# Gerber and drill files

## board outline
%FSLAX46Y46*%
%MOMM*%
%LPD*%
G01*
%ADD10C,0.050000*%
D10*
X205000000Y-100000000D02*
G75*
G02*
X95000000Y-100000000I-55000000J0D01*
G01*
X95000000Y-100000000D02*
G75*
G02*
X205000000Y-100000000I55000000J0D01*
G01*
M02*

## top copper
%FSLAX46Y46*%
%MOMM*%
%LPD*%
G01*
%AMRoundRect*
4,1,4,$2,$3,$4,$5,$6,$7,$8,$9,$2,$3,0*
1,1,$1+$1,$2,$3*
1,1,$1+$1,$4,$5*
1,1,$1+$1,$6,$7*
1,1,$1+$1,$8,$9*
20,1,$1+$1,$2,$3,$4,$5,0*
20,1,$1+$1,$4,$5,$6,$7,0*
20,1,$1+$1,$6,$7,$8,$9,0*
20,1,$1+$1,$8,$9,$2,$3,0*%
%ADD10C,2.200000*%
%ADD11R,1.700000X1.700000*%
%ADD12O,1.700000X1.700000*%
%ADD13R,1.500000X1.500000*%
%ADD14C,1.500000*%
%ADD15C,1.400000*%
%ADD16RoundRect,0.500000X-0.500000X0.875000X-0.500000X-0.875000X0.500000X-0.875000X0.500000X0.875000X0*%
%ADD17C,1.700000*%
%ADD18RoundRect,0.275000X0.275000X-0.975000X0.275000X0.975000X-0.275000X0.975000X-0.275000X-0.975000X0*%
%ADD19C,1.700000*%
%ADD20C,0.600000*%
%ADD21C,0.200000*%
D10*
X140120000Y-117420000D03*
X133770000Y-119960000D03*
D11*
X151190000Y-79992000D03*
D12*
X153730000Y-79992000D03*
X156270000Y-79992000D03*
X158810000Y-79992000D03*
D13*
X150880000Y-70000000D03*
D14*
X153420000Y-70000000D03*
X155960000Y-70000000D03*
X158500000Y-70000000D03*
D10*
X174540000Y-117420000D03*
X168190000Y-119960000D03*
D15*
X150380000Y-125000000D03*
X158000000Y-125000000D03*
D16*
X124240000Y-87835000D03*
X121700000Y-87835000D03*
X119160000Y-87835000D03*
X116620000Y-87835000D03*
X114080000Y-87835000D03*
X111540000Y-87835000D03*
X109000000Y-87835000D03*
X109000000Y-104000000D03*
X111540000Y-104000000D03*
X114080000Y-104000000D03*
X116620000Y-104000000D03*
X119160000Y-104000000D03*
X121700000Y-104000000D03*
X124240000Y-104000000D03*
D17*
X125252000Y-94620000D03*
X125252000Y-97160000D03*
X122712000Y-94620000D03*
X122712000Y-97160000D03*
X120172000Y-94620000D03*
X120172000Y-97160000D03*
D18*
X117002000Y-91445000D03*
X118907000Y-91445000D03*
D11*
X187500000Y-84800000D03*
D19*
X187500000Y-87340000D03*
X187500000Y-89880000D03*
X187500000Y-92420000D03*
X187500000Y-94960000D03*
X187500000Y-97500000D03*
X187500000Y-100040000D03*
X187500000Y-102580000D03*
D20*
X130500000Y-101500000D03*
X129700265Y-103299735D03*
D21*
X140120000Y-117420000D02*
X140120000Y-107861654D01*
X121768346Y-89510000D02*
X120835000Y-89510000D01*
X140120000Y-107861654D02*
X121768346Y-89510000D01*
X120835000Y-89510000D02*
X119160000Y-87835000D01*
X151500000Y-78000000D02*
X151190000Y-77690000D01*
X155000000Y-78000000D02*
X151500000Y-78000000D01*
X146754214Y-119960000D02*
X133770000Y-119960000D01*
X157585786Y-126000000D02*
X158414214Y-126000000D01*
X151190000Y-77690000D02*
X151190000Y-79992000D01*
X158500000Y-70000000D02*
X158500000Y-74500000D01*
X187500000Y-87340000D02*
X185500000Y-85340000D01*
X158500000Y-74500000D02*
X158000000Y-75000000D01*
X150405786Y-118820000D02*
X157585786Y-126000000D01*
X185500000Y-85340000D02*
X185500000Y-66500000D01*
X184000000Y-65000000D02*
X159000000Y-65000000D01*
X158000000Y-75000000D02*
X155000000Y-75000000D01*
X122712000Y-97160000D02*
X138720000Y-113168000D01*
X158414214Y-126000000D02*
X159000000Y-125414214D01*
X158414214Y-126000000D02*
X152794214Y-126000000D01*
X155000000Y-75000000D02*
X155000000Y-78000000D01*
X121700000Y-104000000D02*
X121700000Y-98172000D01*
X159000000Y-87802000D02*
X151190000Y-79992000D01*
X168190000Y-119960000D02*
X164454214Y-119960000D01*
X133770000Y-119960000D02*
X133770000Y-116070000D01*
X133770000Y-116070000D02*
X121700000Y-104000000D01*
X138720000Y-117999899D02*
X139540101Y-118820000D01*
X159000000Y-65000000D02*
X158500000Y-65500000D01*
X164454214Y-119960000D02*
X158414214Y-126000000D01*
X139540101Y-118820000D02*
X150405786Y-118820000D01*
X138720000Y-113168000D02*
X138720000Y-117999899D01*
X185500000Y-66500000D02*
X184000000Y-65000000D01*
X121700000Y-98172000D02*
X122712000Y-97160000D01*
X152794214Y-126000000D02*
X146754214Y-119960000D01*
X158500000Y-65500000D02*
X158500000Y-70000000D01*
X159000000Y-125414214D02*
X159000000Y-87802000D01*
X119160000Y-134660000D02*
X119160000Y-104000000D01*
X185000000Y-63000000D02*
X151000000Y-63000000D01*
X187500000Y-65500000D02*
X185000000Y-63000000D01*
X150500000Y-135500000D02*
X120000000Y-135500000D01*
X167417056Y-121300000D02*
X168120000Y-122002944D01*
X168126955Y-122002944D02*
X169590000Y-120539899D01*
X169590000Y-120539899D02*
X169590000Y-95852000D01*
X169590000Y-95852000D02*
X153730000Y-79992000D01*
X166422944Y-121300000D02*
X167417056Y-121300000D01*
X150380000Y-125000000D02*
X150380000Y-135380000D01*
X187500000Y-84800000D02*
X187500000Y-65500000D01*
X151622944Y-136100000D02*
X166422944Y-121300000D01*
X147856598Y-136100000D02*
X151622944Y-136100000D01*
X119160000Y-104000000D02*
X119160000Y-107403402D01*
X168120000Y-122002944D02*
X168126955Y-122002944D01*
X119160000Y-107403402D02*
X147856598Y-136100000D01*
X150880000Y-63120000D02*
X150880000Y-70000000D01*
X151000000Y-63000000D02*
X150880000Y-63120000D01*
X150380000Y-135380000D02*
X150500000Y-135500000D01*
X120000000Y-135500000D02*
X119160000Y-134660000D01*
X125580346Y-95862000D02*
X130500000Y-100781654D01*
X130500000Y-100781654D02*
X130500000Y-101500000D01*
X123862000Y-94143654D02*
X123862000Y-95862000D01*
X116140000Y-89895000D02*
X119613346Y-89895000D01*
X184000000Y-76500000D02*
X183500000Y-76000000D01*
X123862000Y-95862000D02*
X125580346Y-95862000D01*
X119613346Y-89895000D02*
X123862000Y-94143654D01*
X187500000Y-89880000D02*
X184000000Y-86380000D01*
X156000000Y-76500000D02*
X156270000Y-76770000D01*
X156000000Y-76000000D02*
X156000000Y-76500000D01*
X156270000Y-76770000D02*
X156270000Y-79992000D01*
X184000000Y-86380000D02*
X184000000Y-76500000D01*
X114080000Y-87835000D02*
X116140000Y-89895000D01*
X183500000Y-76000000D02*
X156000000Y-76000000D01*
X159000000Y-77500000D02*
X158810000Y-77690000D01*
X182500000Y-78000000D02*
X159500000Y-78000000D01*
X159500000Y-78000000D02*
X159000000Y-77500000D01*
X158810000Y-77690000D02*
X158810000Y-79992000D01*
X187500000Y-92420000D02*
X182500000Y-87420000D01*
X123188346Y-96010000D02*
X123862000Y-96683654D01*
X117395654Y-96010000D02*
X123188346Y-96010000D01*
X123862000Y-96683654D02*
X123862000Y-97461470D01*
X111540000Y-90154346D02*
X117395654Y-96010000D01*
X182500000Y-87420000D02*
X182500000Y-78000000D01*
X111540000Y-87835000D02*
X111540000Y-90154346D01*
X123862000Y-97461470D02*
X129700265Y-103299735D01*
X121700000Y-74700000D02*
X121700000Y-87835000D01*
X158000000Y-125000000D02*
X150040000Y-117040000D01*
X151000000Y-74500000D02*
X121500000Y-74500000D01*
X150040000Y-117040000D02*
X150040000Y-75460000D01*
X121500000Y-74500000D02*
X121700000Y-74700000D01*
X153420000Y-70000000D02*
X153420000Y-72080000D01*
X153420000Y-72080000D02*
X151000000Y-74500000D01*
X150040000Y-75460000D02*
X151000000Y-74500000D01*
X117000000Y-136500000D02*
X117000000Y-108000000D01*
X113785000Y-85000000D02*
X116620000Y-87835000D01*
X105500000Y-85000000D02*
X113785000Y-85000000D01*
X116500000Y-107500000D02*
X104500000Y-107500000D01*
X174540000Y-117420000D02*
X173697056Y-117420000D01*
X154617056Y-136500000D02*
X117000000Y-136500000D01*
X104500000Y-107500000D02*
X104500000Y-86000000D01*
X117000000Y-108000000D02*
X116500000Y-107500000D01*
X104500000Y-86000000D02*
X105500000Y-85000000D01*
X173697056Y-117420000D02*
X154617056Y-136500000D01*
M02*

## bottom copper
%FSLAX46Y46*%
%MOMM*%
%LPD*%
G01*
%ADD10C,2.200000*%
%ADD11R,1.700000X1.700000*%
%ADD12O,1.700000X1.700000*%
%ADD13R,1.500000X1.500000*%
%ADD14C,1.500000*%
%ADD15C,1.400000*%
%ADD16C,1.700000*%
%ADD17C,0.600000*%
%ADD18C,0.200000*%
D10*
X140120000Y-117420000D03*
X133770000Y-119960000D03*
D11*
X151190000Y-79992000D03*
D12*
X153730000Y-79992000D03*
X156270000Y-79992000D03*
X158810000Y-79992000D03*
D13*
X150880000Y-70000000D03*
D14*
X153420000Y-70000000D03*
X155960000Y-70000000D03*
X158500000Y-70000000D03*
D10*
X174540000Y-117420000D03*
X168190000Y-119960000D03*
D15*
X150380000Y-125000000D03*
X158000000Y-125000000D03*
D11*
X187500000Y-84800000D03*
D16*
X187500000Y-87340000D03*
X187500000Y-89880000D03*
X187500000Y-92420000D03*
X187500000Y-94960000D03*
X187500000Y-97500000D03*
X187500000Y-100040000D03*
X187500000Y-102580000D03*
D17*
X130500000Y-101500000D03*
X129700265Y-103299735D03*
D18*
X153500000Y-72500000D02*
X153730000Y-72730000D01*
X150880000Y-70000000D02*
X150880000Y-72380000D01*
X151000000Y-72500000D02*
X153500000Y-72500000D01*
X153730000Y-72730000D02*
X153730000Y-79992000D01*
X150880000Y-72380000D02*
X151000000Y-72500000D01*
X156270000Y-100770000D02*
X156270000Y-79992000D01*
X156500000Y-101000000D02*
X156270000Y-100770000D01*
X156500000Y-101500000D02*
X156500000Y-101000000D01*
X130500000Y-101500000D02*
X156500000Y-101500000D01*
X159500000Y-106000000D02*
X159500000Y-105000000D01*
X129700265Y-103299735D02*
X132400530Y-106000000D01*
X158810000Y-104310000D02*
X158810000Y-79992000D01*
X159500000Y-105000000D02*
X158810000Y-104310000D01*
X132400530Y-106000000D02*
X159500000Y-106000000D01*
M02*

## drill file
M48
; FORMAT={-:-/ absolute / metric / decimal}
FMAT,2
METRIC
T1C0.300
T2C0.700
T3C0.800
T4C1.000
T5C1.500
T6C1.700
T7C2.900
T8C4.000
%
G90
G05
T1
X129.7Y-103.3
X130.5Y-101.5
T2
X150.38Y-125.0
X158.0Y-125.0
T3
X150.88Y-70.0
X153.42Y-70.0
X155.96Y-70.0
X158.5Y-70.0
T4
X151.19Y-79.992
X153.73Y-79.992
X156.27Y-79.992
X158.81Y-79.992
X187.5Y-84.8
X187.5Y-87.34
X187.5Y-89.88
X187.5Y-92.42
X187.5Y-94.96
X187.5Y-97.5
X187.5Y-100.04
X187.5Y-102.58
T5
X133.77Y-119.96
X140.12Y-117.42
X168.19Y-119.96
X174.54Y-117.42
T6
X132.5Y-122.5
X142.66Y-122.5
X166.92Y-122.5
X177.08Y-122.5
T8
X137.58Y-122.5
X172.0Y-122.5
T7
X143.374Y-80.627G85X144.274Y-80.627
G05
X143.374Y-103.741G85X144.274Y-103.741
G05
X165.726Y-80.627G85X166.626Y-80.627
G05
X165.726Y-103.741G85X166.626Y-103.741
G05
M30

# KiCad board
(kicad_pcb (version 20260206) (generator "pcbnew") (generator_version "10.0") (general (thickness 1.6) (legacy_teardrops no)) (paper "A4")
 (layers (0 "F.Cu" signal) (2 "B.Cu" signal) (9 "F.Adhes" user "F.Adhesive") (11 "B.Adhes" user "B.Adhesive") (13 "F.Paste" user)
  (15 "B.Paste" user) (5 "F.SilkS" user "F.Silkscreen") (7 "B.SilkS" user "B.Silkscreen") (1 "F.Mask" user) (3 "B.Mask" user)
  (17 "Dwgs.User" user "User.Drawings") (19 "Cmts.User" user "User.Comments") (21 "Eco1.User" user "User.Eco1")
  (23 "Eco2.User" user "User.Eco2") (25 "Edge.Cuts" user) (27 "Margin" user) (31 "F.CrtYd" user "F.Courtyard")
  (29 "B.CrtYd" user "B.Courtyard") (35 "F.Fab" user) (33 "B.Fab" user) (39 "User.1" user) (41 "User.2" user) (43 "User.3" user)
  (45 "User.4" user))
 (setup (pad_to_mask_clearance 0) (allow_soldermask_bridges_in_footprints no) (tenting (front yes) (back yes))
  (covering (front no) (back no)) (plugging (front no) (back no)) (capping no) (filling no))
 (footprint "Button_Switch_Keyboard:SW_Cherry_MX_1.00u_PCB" (layer "F.Cu") (at 140.12 117.42)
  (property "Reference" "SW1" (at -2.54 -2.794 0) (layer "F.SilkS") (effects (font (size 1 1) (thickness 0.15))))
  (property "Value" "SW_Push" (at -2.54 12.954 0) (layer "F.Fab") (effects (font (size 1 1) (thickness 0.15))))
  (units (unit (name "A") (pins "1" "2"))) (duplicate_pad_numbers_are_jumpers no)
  (pad "" np_thru_hole circle (at -7.62 5.08) (size 1.7 1.7) (drill 1.7) (layers "*.Cu" "*.Mask"))
  (pad "" np_thru_hole circle (at -2.54 5.08) (size 4 4) (drill 4) (layers "*.Cu" "*.Mask"))
  (pad "" np_thru_hole circle (at 2.54 5.08) (size 1.7 1.7) (drill 1.7) (layers "*.Cu" "*.Mask"))
  (pad "1" thru_hole circle (at 0 0) (size 2.2 2.2) (drill 1.5) (layers "*.Cu" "*.Mask") (remove_unused_layers no) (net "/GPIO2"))
  (pad "2" thru_hole circle (at -6.35 2.54) (size 2.2 2.2) (drill 1.5) (layers "*.Cu" "*.Mask") (remove_unused_layers no) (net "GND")))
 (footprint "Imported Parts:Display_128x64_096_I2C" (layer "F.Cu") (at 155 79.992)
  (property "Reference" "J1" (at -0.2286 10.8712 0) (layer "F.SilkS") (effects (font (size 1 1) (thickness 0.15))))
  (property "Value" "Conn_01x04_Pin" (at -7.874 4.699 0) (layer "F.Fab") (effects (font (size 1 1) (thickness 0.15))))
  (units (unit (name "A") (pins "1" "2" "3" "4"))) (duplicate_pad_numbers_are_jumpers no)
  (pad "" np_thru_hole oval (at -11.176 0.635) (size 3.8 2.9) (drill oval 3.8 2.9) (layers "*.Cu" "*.Mask"))
  (pad "" np_thru_hole oval (at -11.176 23.749) (size 3.8 2.9) (drill oval 3.8 2.9) (layers "*.Cu" "*.Mask"))
  (pad "" np_thru_hole oval (at 11.176 0.635) (size 3.8 2.9) (drill oval 3.8 2.9) (layers "*.Cu" "*.Mask"))
  (pad "" np_thru_hole oval (at 11.176 23.749) (size 3.8 2.9) (drill oval 3.8 2.9) (layers "*.Cu" "*.Mask"))
  (pad "1" thru_hole rect (at -3.81 0 90) (size 1.7 1.7) (drill 1) (layers "*.Cu" "*.Mask") (remove_unused_layers no) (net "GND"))
  (pad "2" thru_hole oval (at -1.27 0 90) (size 1.7 1.7) (drill 1) (layers "*.Cu" "*.Mask") (remove_unused_layers no) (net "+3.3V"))
  (pad "3" thru_hole oval (at 1.27 0 90) (size 1.7 1.7) (drill 1) (layers "*.Cu" "*.Mask") (remove_unused_layers no) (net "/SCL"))
  (pad "4" thru_hole oval (at 3.81 0 90) (size 1.7 1.7) (drill 1) (layers "*.Cu" "*.Mask") (remove_unused_layers no) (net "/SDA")))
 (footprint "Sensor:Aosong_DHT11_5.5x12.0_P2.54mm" (layer "F.Cu") (at 150.88 70 90)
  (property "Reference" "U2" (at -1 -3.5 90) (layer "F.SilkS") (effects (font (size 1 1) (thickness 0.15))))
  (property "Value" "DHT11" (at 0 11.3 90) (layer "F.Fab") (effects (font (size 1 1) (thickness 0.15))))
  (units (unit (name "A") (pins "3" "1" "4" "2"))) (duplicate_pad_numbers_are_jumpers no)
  (pad "1" thru_hole rect (at 0 0 90) (size 1.5 1.5) (drill 0.8) (layers "*.Cu" "*.Mask") (remove_unused_layers no) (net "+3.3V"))
  (pad "2" thru_hole circle (at 0 2.54 90) (size 1.5 1.5) (drill 0.8) (layers "*.Cu" "*.Mask") (remove_unused_layers no) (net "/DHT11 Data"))
  (pad "3" thru_hole circle (at 0 5.08 90) (size 1.5 1.5) (drill 0.8) (layers "*.Cu" "*.Mask") (remove_unused_layers no)
   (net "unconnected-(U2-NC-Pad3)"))
  (pad "4" thru_hole circle (at 0 7.62 90) (size 1.5 1.5) (drill 0.8) (layers "*.Cu" "*.Mask") (remove_unused_layers no) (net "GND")))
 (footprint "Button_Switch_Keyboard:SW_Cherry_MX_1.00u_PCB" (layer "F.Cu") (at 174.54 117.42)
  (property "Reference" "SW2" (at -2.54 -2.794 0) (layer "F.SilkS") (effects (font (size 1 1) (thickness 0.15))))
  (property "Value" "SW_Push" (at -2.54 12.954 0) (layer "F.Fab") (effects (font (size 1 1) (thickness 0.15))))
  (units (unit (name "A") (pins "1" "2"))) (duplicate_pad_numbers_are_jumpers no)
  (pad "" np_thru_hole circle (at -7.62 5.08) (size 1.7 1.7) (drill 1.7) (layers "*.Cu" "*.Mask"))
  (pad "" np_thru_hole circle (at -2.54 5.08) (size 4 4) (drill 4) (layers "*.Cu" "*.Mask"))
  (pad "" np_thru_hole circle (at 2.54 5.08) (size 1.7 1.7) (drill 1.7) (layers "*.Cu" "*.Mask"))
  (pad "1" thru_hole circle (at 0 0) (size 2.2 2.2) (drill 1.5) (layers "*.Cu" "*.Mask") (remove_unused_layers no) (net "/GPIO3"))
  (pad "2" thru_hole circle (at -6.35 2.54) (size 2.2 2.2) (drill 1.5) (layers "*.Cu" "*.Mask") (remove_unused_layers no) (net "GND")))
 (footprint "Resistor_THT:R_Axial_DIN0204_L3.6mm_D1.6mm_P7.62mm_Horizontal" (layer "F.Cu") (at 150.38 125)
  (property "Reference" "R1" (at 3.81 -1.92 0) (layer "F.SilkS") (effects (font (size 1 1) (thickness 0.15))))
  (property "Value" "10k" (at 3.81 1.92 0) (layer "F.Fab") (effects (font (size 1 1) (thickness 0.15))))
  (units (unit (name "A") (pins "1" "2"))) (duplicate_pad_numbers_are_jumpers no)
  (pad "1" thru_hole circle (at 0 0) (size 1.4 1.4) (drill 0.7) (layers "*.Cu" "*.Mask") (remove_unused_layers no) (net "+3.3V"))
  (pad "2" thru_hole circle (at 7.62 0) (size 1.4 1.4) (drill 0.7) (layers "*.Cu" "*.Mask") (remove_unused_layers no) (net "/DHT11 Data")))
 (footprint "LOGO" (layer "F.Cu") (at 133 62)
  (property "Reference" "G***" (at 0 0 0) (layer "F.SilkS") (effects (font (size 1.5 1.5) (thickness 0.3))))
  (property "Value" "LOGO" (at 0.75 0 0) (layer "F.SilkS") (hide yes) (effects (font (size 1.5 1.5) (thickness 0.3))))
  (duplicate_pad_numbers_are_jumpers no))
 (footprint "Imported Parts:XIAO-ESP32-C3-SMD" (layer "F.Cu") (at 106.12 87 -90)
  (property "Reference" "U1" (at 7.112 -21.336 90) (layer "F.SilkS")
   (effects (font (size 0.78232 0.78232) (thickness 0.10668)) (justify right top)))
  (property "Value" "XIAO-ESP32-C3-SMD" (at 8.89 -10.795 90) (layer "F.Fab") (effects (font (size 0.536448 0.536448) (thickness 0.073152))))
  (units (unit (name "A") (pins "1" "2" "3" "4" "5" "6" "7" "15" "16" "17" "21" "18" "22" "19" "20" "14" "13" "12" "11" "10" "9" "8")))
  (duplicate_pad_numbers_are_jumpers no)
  (pad "1" smd roundrect (at 0.835 -18.12 270) (size 2.75 2) (layers "F.Cu" "F.Mask" "F.Paste") (roundrect_rratio 0.25)
   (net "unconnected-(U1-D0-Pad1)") (solder_mask_margin 0.0508) (thermal_bridge_angle 45))
  (pad "2" smd roundrect (at 0.835 -15.58 270) (size 2.75 2) (layers "F.Cu" "F.Mask" "F.Paste") (roundrect_rratio 0.25) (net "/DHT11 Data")
   (solder_mask_margin 0.0508) (thermal_bridge_angle 45))
  (pad "3" smd roundrect (at 0.835 -13.04 270) (size 2.75 2) (layers "F.Cu" "F.Mask" "F.Paste") (roundrect_rratio 0.25) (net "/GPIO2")
   (solder_mask_margin 0.0508) (thermal_bridge_angle 45))
  (pad "4" smd roundrect (at 0.835 -10.5 270) (size 2.75 2) (layers "F.Cu" "F.Mask" "F.Paste") (roundrect_rratio 0.25) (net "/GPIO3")
   (solder_mask_margin 0.0508) (thermal_bridge_angle 45))
  (pad "5" smd roundrect (at 0.835 -7.96 270) (size 2.75 2) (layers "F.Cu" "F.Mask" "F.Paste") (roundrect_rratio 0.25) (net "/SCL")
   (solder_mask_margin 0.0508) (thermal_bridge_angle 45))
  (pad "6" smd roundrect (at 0.835 -5.42 270) (size 2.75 2) (layers "F.Cu" "F.Mask" "F.Paste") (roundrect_rratio 0.25) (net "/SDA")
   (solder_mask_margin 0.0508) (thermal_bridge_angle 45))
  (pad "7" smd roundrect (at 0.835 -2.88 270) (size 2.75 2) (layers "F.Cu" "F.Mask" "F.Paste") (roundrect_rratio 0.25)
   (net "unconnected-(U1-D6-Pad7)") (solder_mask_margin 0.0508) (thermal_bridge_angle 45))
  (pad "8" smd roundrect (at 17 -2.88 270) (size 2.75 2) (layers "F.Cu" "F.Mask" "F.Paste") (roundrect_rratio 0.25)
   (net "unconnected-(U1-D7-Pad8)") (solder_mask_margin 0.0508) (thermal_bridge_angle 45))
  (pad "9" smd roundrect (at 17 -5.42 270) (size 2.75 2) (layers "F.Cu" "F.Mask" "F.Paste") (roundrect_rratio 0.25)
   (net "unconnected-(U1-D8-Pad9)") (solder_mask_margin 0.0508) (thermal_bridge_angle 45))
  (pad "10" smd roundrect (at 17 -7.96 270) (size 2.75 2) (layers "F.Cu" "F.Mask" "F.Paste") (roundrect_rratio 0.25)
   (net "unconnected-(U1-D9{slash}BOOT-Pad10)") (solder_mask_margin 0.0508) (thermal_bridge_angle 45))
  (pad "11" smd roundrect (at 17 -10.5 270) (size 2.75 2) (layers "F.Cu" "F.Mask" "F.Paste") (roundrect_rratio 0.25)
   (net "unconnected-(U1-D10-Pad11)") (solder_mask_margin 0.0508) (thermal_bridge_angle 45))
  (pad "12" smd roundrect (at 17 -13.04 270) (size 2.75 2) (layers "F.Cu" "F.Mask" "F.Paste") (roundrect_rratio 0.25) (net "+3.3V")
   (solder_mask_margin 0.0508) (thermal_bridge_angle 45))
  (pad "13" smd roundrect (at 17 -15.58 270) (size 2.75 2) (layers "F.Cu" "F.Mask" "F.Paste") (roundrect_rratio 0.25) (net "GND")
   (solder_mask_margin 0.0508) (thermal_bridge_angle 45))
  (pad "14" smd roundrect (at 17 -18.12 270) (size 2.75 2) (layers "F.Cu" "F.Mask" "F.Paste") (roundrect_rratio 0.25) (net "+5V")
   (solder_mask_margin 0.0508) (thermal_bridge_angle 45))
  (pad "15" smd circle (at 7.62 -19.132 270) (size 1.7 1.7) (layers "F.Cu" "F.Mask" "F.Paste") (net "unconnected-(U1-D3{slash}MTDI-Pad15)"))
  (pad "16" smd circle (at 10.16 -19.132 270) (size 1.7 1.7) (layers "F.Cu" "F.Mask" "F.Paste") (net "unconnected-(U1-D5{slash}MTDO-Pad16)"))
  (pad "17" smd circle (at 7.62 -16.592 270) (size 1.7 1.7) (layers "F.Cu" "F.Mask" "F.Paste") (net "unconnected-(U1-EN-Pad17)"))
  (pad "18" smd circle (at 10.16 -16.592 270) (size 1.7 1.7) (layers "F.Cu" "F.Mask" "F.Paste") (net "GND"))
  (pad "19" smd circle (at 7.62 -14.052 270) (size 1.7 1.7) (layers "F.Cu" "F.Mask" "F.Paste") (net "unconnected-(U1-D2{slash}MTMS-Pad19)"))
  (pad "20" smd circle (at 10.16 -14.052 270) (size 1.7 1.7) (layers "F.Cu" "F.Mask" "F.Paste") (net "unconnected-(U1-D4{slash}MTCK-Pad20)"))
  (pad "21" smd roundrect (at 4.445 -10.882 90) (size 2.5 1.1) (layers "F.Cu" "F.Mask" "F.Paste") (roundrect_rratio 0.25)
   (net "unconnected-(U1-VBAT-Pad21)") (thermal_bridge_angle 45))
  (pad "22" smd roundrect (at 4.445 -12.787 90) (size 2.5 1.1) (layers "F.Cu" "F.Mask" "F.Paste") (roundrect_rratio 0.25)
   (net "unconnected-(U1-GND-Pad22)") (thermal_bridge_angle 45)))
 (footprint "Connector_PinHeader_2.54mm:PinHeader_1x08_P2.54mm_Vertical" (layer "F.Cu") (at 187.5 84.8)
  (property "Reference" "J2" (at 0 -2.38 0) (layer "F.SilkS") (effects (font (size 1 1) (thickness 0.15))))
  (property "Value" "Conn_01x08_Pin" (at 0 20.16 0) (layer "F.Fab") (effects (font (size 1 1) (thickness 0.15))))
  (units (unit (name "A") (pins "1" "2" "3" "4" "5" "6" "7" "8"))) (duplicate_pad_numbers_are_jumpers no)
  (pad "1" thru_hole rect (at 0 0) (size 1.7 1.7) (drill 1) (layers "*.Cu" "*.Mask") (remove_unused_layers no) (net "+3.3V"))
  (pad "2" thru_hole circle (at 0 2.54) (size 1.7 1.7) (drill 1) (layers "*.Cu" "*.Mask") (remove_unused_layers no) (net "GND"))
  (pad "3" thru_hole circle (at 0 5.08) (size 1.7 1.7) (drill 1) (layers "*.Cu" "*.Mask") (remove_unused_layers no) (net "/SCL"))
  (pad "4" thru_hole circle (at 0 7.62) (size 1.7 1.7) (drill 1) (layers "*.Cu" "*.Mask") (remove_unused_layers no) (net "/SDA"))
  (pad "5" thru_hole circle (at 0 10.16) (size 1.7 1.7) (drill 1) (layers "*.Cu" "*.Mask") (remove_unused_layers no)
   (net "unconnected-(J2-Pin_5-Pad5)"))
  (pad "6" thru_hole circle (at 0 12.7) (size 1.7 1.7) (drill 1) (layers "*.Cu" "*.Mask") (remove_unused_layers no)
   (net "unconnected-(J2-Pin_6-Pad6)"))
  (pad "7" thru_hole circle (at 0 15.24) (size 1.7 1.7) (drill 1) (layers "*.Cu" "*.Mask") (remove_unused_layers no)
   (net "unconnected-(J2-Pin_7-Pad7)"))
  (pad "8" thru_hole circle (at 0 17.78) (size 1.7 1.7) (drill 1) (layers "*.Cu" "*.Mask") (remove_unused_layers no)
   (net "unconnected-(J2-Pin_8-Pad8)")))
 (gr_circle (center 150 100) (end 205 100) (stroke (width 0.05) (type solid)) (fill no) (layer "Edge.Cuts"))
 (segment (start 140.12 117.42) (end 140.12 107.861654) (width 0.2) (layer "F.Cu") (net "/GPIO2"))
 (segment (start 121.768346 89.51) (end 120.835 89.51) (width 0.2) (layer "F.Cu") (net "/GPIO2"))
 (segment (start 140.12 107.861654) (end 121.768346 89.51) (width 0.2) (layer "F.Cu") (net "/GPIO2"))
 (segment (start 120.835 89.51) (end 119.16 87.835) (width 0.2) (layer "F.Cu") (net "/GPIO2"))
 (segment (start 151.5 78) (end 151.19 77.69) (width 0.2) (layer "F.Cu") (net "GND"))
 (segment (start 155 78) (end 151.5 78) (width 0.2) (layer "F.Cu") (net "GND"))
 (segment (start 146.754214 119.96) (end 133.77 119.96) (width 0.2) (layer "F.Cu") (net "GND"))
 (segment (start 157.585786 126) (end 158.414214 126) (width 0.2) (layer "F.Cu") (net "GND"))
 (segment (start 151.19 77.69) (end 151.19 79.992) (width 0.2) (layer "F.Cu") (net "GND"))
 (segment (start 158.5 70) (end 158.5 74.5) (width 0.2) (layer "F.Cu") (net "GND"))
 (segment (start 187.5 87.34) (end 185.5 85.34) (width 0.2) (layer "F.Cu") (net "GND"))
 (segment (start 158.5 74.5) (end 158 75) (width 0.2) (layer "F.Cu") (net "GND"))
 (segment (start 150.405786 118.82) (end 157.585786 126) (width 0.2) (layer "F.Cu") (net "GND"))
 (segment (start 185.5 85.34) (end 185.5 66.5) (width 0.2) (layer "F.Cu") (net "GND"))
 (segment (start 184 65) (end 159 65) (width 0.2) (layer "F.Cu") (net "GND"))
 (segment (start 158 75) (end 155 75) (width 0.2) (layer "F.Cu") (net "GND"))
 (segment (start 122.712 97.16) (end 138.72 113.168) (width 0.2) (layer "F.Cu") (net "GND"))
 (segment (start 158.414214 126) (end 159 125.414214) (width 0.2) (layer "F.Cu") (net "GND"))
 (segment (start 158.414214 126) (end 152.794214 126) (width 0.2) (layer "F.Cu") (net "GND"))
 (segment (start 155 75) (end 155 78) (width 0.2) (layer "F.Cu") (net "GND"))
 (segment (start 121.7 104) (end 121.7 98.172) (width 0.2) (layer "F.Cu") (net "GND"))
 (segment (start 159 87.802) (end 151.19 79.992) (width 0.2) (layer "F.Cu") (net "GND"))
 (segment (start 168.19 119.96) (end 164.454214 119.96) (width 0.2) (layer "F.Cu") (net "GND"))
 (segment (start 133.77 119.96) (end 133.77 116.07) (width 0.2) (layer "F.Cu") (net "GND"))
 (segment (start 133.77 116.07) (end 121.7 104) (width 0.2) (layer "F.Cu") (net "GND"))
 (segment (start 138.72 117.999899) (end 139.540101 118.82) (width 0.2) (layer "F.Cu") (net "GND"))
 (segment (start 159 65) (end 158.5 65.5) (width 0.2) (layer "F.Cu") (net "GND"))
 (segment (start 164.454214 119.96) (end 158.414214 126) (width 0.2) (layer "F.Cu") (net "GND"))
 (segment (start 139.540101 118.82) (end 150.405786 118.82) (width 0.2) (layer "F.Cu") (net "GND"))
 (segment (start 138.72 113.168) (end 138.72 117.999899) (width 0.2) (layer "F.Cu") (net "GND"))
 (segment (start 185.5 66.5) (end 184 65) (width 0.2) (layer "F.Cu") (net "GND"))
 (segment (start 121.7 98.172) (end 122.712 97.16) (width 0.2) (layer "F.Cu") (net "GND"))
 (segment (start 152.794214 126) (end 146.754214 119.96) (width 0.2) (layer "F.Cu") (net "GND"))
 (segment (start 158.5 65.5) (end 158.5 70) (width 0.2) (layer "F.Cu") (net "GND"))
 (segment (start 159 125.414214) (end 159 87.802) (width 0.2) (layer "F.Cu") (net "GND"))
 (segment (start 119.16 134.66) (end 119.16 104) (width 0.2) (layer "F.Cu") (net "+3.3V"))
 (segment (start 185 63) (end 151 63) (width 0.2) (layer "F.Cu") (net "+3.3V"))
 (segment (start 187.5 65.5) (end 185 63) (width 0.2) (layer "F.Cu") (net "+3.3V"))
 (segment (start 150.5 135.5) (end 120 135.5) (width 0.2) (layer "F.Cu") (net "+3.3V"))
 (segment (start 167.417056 121.3) (end 168.12 122.002944) (width 0.2) (layer "F.Cu") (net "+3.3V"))
 (segment (start 168.126955 122.002944) (end 169.59 120.539899) (width 0.2) (layer "F.Cu") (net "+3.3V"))
 (segment (start 169.59 120.539899) (end 169.59 95.852) (width 0.2) (layer "F.Cu") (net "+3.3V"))
 (segment (start 169.59 95.852) (end 153.73 79.992) (width 0.2) (layer "F.Cu") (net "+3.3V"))
 (segment (start 166.422944 121.3) (end 167.417056 121.3) (width 0.2) (layer "F.Cu") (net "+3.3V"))
 (segment (start 150.38 125) (end 150.38 135.38) (width 0.2) (layer "F.Cu") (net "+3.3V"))
 (segment (start 187.5 84.8) (end 187.5 65.5) (width 0.2) (layer "F.Cu") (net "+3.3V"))
 (segment (start 151.622944 136.1) (end 166.422944 121.3) (width 0.2) (layer "F.Cu") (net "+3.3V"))
 (segment (start 147.856598 136.1) (end 151.622944 136.1) (width 0.2) (layer "F.Cu") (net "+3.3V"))
 (segment (start 119.16 104) (end 119.16 107.403402) (width 0.2) (layer "F.Cu") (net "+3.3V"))
 (segment (start 168.12 122.002944) (end 168.126955 122.002944) (width 0.2) (layer "F.Cu") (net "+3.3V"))
 (segment (start 119.16 107.403402) (end 147.856598 136.1) (width 0.2) (layer "F.Cu") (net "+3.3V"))
 (segment (start 150.88 63.12) (end 150.88 70) (width 0.2) (layer "F.Cu") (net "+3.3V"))
 (segment (start 151 63) (end 150.88 63.12) (width 0.2) (layer "F.Cu") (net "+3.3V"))
 (segment (start 150.38 135.38) (end 150.5 135.5) (width 0.2) (layer "F.Cu") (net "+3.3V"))
 (segment (start 120 135.5) (end 119.16 134.66) (width 0.2) (layer "F.Cu") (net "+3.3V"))
 (segment (start 153.5 72.5) (end 153.73 72.73) (width 0.2) (layer "B.Cu") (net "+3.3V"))
 (segment (start 150.88 70) (end 150.88 72.38) (width 0.2) (layer "B.Cu") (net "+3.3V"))
 (segment (start 151 72.5) (end 153.5 72.5) (width 0.2) (layer "B.Cu") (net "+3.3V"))
 (segment (start 153.73 72.73) (end 153.73 79.992) (width 0.2) (layer "B.Cu") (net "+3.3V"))
 (segment (start 150.88 72.38) (end 151 72.5) (width 0.2) (layer "B.Cu") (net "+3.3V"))
 (segment (start 125.580346 95.862) (end 130.5 100.781654) (width 0.2) (layer "F.Cu") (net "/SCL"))
 (segment (start 130.5 100.781654) (end 130.5 101.5) (width 0.2) (layer "F.Cu") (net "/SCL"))
 (segment (start 123.862 94.143654) (end 123.862 95.862) (width 0.2) (layer "F.Cu") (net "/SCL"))
 (segment (start 116.14 89.895) (end 119.613346 89.895) (width 0.2) (layer "F.Cu") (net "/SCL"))
 (segment (start 184 76.5) (end 183.5 76) (width 0.2) (layer "F.Cu") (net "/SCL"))
 (segment (start 123.862 95.862) (end 125.580346 95.862) (width 0.2) (layer "F.Cu") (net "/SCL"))
 (segment (start 119.613346 89.895) (end 123.862 94.143654) (width 0.2) (layer "F.Cu") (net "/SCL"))
 (segment (start 187.5 89.88) (end 184 86.38) (width 0.2) (layer "F.Cu") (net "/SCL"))
 (segment (start 156 76.5) (end 156.27 76.77) (width 0.2) (layer "F.Cu") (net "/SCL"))
 (segment (start 156 76) (end 156 76.5) (width 0.2) (layer "F.Cu") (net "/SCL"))
 (segment (start 156.27 76.77) (end 156.27 79.992) (width 0.2) (layer "F.Cu") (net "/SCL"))
 (segment (start 184 86.38) (end 184 76.5) (width 0.2) (layer "F.Cu") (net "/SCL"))
 (segment (start 114.08 87.835) (end 116.14 89.895) (width 0.2) (layer "F.Cu") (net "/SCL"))
 (segment (start 183.5 76) (end 156 76) (width 0.2) (layer "F.Cu") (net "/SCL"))
 (via (at 130.5 101.5) (size 0.6) (drill 0.3) (layers "F.Cu" "B.Cu") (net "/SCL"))
 (segment (start 156.27 100.77) (end 156.27 79.992) (width 0.2) (layer "B.Cu") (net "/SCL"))
 (segment (start 156.5 101) (end 156.27 100.77) (width 0.2) (layer "B.Cu") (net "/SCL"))
 (segment (start 156.5 101.5) (end 156.5 101) (width 0.2) (layer "B.Cu") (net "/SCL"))
 (segment (start 130.5 101.5) (end 156.5 101.5) (width 0.2) (layer "B.Cu") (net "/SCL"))
 (segment (start 159 77.5) (end 158.81 77.69) (width 0.2) (layer "F.Cu") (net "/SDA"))
 (segment (start 182.5 78) (end 159.5 78) (width 0.2) (layer "F.Cu") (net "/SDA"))
 (segment (start 159.5 78) (end 159 77.5) (width 0.2) (layer "F.Cu") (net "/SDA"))
 (segment (start 158.81 77.69) (end 158.81 79.992) (width 0.2) (layer "F.Cu") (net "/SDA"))
 (segment (start 187.5 92.42) (end 182.5 87.42) (width 0.2) (layer "F.Cu") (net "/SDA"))
 (segment (start 123.188346 96.01) (end 123.862 96.683654) (width 0.2) (layer "F.Cu") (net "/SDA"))
 (segment (start 117.395654 96.01) (end 123.188346 96.01) (width 0.2) (layer "F.Cu") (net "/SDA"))
 (segment (start 123.862 96.683654) (end 123.862 97.46147) (width 0.2) (layer "F.Cu") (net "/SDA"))
 (segment (start 111.54 90.154346) (end 117.395654 96.01) (width 0.2) (layer "F.Cu") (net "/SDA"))
 (segment (start 182.5 87.42) (end 182.5 78) (width 0.2) (layer "F.Cu") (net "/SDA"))
 (segment (start 111.54 87.835) (end 111.54 90.154346) (width 0.2) (layer "F.Cu") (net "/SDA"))
 (segment (start 123.862 97.46147) (end 129.700265 103.299735) (width 0.2) (layer "F.Cu") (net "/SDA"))
 (via (at 129.700265 103.299735) (size 0.6) (drill 0.3) (layers "F.Cu" "B.Cu") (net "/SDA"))
 (segment (start 159.5 106) (end 159.5 105) (width 0.2) (layer "B.Cu") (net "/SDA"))
 (segment (start 129.700265 103.299735) (end 132.40053 106) (width 0.2) (layer "B.Cu") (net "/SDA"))
 (segment (start 158.81 104.31) (end 158.81 79.992) (width 0.2) (layer "B.Cu") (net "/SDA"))
 (segment (start 159.5 105) (end 158.81 104.31) (width 0.2) (layer "B.Cu") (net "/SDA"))
 (segment (start 132.40053 106) (end 159.5 106) (width 0.2) (layer "B.Cu") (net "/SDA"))
 (segment (start 121.7 74.7) (end 121.7 87.835) (width 0.2) (layer "F.Cu") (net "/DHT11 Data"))
 (segment (start 158 125) (end 150.04 117.04) (width 0.2) (layer "F.Cu") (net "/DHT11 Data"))
 (segment (start 151 74.5) (end 121.5 74.5) (width 0.2) (layer "F.Cu") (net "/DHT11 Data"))
 (segment (start 150.04 117.04) (end 150.04 75.46) (width 0.2) (layer "F.Cu") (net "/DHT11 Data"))
 (segment (start 121.5 74.5) (end 121.7 74.7) (width 0.2) (layer "F.Cu") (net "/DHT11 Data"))
 (segment (start 153.42 70) (end 153.42 72.08) (width 0.2) (layer "F.Cu") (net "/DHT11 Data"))
 (segment (start 153.42 72.08) (end 151 74.5) (width 0.2) (layer "F.Cu") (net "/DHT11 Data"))
 (segment (start 150.04 75.46) (end 151 74.5) (width 0.2) (layer "F.Cu") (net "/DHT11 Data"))
 (segment (start 117 136.5) (end 117 108) (width 0.2) (layer "F.Cu") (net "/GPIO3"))
 (segment (start 113.785 85) (end 116.62 87.835) (width 0.2) (layer "F.Cu") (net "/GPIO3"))
 (segment (start 105.5 85) (end 113.785 85) (width 0.2) (layer "F.Cu") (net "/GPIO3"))
 (segment (start 116.5 107.5) (end 104.5 107.5) (width 0.2) (layer "F.Cu") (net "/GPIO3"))
 (segment (start 174.54 117.42) (end 173.697056 117.42) (width 0.2) (layer "F.Cu") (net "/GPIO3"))
 (segment (start 154.617056 136.5) (end 117 136.5) (width 0.2) (layer "F.Cu") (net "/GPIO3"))
 (segment (start 104.5 107.5) (end 104.5 86) (width 0.2) (layer "F.Cu") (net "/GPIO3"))
 (segment (start 117 108) (end 116.5 107.5) (width 0.2) (layer "F.Cu") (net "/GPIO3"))
 (segment (start 104.5 86) (end 105.5 85) (width 0.2) (layer "F.Cu") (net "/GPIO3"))
 (segment (start 173.697056 117.42) (end 154.617056 136.5) (width 0.2) (layer "F.Cu") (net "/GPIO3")))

